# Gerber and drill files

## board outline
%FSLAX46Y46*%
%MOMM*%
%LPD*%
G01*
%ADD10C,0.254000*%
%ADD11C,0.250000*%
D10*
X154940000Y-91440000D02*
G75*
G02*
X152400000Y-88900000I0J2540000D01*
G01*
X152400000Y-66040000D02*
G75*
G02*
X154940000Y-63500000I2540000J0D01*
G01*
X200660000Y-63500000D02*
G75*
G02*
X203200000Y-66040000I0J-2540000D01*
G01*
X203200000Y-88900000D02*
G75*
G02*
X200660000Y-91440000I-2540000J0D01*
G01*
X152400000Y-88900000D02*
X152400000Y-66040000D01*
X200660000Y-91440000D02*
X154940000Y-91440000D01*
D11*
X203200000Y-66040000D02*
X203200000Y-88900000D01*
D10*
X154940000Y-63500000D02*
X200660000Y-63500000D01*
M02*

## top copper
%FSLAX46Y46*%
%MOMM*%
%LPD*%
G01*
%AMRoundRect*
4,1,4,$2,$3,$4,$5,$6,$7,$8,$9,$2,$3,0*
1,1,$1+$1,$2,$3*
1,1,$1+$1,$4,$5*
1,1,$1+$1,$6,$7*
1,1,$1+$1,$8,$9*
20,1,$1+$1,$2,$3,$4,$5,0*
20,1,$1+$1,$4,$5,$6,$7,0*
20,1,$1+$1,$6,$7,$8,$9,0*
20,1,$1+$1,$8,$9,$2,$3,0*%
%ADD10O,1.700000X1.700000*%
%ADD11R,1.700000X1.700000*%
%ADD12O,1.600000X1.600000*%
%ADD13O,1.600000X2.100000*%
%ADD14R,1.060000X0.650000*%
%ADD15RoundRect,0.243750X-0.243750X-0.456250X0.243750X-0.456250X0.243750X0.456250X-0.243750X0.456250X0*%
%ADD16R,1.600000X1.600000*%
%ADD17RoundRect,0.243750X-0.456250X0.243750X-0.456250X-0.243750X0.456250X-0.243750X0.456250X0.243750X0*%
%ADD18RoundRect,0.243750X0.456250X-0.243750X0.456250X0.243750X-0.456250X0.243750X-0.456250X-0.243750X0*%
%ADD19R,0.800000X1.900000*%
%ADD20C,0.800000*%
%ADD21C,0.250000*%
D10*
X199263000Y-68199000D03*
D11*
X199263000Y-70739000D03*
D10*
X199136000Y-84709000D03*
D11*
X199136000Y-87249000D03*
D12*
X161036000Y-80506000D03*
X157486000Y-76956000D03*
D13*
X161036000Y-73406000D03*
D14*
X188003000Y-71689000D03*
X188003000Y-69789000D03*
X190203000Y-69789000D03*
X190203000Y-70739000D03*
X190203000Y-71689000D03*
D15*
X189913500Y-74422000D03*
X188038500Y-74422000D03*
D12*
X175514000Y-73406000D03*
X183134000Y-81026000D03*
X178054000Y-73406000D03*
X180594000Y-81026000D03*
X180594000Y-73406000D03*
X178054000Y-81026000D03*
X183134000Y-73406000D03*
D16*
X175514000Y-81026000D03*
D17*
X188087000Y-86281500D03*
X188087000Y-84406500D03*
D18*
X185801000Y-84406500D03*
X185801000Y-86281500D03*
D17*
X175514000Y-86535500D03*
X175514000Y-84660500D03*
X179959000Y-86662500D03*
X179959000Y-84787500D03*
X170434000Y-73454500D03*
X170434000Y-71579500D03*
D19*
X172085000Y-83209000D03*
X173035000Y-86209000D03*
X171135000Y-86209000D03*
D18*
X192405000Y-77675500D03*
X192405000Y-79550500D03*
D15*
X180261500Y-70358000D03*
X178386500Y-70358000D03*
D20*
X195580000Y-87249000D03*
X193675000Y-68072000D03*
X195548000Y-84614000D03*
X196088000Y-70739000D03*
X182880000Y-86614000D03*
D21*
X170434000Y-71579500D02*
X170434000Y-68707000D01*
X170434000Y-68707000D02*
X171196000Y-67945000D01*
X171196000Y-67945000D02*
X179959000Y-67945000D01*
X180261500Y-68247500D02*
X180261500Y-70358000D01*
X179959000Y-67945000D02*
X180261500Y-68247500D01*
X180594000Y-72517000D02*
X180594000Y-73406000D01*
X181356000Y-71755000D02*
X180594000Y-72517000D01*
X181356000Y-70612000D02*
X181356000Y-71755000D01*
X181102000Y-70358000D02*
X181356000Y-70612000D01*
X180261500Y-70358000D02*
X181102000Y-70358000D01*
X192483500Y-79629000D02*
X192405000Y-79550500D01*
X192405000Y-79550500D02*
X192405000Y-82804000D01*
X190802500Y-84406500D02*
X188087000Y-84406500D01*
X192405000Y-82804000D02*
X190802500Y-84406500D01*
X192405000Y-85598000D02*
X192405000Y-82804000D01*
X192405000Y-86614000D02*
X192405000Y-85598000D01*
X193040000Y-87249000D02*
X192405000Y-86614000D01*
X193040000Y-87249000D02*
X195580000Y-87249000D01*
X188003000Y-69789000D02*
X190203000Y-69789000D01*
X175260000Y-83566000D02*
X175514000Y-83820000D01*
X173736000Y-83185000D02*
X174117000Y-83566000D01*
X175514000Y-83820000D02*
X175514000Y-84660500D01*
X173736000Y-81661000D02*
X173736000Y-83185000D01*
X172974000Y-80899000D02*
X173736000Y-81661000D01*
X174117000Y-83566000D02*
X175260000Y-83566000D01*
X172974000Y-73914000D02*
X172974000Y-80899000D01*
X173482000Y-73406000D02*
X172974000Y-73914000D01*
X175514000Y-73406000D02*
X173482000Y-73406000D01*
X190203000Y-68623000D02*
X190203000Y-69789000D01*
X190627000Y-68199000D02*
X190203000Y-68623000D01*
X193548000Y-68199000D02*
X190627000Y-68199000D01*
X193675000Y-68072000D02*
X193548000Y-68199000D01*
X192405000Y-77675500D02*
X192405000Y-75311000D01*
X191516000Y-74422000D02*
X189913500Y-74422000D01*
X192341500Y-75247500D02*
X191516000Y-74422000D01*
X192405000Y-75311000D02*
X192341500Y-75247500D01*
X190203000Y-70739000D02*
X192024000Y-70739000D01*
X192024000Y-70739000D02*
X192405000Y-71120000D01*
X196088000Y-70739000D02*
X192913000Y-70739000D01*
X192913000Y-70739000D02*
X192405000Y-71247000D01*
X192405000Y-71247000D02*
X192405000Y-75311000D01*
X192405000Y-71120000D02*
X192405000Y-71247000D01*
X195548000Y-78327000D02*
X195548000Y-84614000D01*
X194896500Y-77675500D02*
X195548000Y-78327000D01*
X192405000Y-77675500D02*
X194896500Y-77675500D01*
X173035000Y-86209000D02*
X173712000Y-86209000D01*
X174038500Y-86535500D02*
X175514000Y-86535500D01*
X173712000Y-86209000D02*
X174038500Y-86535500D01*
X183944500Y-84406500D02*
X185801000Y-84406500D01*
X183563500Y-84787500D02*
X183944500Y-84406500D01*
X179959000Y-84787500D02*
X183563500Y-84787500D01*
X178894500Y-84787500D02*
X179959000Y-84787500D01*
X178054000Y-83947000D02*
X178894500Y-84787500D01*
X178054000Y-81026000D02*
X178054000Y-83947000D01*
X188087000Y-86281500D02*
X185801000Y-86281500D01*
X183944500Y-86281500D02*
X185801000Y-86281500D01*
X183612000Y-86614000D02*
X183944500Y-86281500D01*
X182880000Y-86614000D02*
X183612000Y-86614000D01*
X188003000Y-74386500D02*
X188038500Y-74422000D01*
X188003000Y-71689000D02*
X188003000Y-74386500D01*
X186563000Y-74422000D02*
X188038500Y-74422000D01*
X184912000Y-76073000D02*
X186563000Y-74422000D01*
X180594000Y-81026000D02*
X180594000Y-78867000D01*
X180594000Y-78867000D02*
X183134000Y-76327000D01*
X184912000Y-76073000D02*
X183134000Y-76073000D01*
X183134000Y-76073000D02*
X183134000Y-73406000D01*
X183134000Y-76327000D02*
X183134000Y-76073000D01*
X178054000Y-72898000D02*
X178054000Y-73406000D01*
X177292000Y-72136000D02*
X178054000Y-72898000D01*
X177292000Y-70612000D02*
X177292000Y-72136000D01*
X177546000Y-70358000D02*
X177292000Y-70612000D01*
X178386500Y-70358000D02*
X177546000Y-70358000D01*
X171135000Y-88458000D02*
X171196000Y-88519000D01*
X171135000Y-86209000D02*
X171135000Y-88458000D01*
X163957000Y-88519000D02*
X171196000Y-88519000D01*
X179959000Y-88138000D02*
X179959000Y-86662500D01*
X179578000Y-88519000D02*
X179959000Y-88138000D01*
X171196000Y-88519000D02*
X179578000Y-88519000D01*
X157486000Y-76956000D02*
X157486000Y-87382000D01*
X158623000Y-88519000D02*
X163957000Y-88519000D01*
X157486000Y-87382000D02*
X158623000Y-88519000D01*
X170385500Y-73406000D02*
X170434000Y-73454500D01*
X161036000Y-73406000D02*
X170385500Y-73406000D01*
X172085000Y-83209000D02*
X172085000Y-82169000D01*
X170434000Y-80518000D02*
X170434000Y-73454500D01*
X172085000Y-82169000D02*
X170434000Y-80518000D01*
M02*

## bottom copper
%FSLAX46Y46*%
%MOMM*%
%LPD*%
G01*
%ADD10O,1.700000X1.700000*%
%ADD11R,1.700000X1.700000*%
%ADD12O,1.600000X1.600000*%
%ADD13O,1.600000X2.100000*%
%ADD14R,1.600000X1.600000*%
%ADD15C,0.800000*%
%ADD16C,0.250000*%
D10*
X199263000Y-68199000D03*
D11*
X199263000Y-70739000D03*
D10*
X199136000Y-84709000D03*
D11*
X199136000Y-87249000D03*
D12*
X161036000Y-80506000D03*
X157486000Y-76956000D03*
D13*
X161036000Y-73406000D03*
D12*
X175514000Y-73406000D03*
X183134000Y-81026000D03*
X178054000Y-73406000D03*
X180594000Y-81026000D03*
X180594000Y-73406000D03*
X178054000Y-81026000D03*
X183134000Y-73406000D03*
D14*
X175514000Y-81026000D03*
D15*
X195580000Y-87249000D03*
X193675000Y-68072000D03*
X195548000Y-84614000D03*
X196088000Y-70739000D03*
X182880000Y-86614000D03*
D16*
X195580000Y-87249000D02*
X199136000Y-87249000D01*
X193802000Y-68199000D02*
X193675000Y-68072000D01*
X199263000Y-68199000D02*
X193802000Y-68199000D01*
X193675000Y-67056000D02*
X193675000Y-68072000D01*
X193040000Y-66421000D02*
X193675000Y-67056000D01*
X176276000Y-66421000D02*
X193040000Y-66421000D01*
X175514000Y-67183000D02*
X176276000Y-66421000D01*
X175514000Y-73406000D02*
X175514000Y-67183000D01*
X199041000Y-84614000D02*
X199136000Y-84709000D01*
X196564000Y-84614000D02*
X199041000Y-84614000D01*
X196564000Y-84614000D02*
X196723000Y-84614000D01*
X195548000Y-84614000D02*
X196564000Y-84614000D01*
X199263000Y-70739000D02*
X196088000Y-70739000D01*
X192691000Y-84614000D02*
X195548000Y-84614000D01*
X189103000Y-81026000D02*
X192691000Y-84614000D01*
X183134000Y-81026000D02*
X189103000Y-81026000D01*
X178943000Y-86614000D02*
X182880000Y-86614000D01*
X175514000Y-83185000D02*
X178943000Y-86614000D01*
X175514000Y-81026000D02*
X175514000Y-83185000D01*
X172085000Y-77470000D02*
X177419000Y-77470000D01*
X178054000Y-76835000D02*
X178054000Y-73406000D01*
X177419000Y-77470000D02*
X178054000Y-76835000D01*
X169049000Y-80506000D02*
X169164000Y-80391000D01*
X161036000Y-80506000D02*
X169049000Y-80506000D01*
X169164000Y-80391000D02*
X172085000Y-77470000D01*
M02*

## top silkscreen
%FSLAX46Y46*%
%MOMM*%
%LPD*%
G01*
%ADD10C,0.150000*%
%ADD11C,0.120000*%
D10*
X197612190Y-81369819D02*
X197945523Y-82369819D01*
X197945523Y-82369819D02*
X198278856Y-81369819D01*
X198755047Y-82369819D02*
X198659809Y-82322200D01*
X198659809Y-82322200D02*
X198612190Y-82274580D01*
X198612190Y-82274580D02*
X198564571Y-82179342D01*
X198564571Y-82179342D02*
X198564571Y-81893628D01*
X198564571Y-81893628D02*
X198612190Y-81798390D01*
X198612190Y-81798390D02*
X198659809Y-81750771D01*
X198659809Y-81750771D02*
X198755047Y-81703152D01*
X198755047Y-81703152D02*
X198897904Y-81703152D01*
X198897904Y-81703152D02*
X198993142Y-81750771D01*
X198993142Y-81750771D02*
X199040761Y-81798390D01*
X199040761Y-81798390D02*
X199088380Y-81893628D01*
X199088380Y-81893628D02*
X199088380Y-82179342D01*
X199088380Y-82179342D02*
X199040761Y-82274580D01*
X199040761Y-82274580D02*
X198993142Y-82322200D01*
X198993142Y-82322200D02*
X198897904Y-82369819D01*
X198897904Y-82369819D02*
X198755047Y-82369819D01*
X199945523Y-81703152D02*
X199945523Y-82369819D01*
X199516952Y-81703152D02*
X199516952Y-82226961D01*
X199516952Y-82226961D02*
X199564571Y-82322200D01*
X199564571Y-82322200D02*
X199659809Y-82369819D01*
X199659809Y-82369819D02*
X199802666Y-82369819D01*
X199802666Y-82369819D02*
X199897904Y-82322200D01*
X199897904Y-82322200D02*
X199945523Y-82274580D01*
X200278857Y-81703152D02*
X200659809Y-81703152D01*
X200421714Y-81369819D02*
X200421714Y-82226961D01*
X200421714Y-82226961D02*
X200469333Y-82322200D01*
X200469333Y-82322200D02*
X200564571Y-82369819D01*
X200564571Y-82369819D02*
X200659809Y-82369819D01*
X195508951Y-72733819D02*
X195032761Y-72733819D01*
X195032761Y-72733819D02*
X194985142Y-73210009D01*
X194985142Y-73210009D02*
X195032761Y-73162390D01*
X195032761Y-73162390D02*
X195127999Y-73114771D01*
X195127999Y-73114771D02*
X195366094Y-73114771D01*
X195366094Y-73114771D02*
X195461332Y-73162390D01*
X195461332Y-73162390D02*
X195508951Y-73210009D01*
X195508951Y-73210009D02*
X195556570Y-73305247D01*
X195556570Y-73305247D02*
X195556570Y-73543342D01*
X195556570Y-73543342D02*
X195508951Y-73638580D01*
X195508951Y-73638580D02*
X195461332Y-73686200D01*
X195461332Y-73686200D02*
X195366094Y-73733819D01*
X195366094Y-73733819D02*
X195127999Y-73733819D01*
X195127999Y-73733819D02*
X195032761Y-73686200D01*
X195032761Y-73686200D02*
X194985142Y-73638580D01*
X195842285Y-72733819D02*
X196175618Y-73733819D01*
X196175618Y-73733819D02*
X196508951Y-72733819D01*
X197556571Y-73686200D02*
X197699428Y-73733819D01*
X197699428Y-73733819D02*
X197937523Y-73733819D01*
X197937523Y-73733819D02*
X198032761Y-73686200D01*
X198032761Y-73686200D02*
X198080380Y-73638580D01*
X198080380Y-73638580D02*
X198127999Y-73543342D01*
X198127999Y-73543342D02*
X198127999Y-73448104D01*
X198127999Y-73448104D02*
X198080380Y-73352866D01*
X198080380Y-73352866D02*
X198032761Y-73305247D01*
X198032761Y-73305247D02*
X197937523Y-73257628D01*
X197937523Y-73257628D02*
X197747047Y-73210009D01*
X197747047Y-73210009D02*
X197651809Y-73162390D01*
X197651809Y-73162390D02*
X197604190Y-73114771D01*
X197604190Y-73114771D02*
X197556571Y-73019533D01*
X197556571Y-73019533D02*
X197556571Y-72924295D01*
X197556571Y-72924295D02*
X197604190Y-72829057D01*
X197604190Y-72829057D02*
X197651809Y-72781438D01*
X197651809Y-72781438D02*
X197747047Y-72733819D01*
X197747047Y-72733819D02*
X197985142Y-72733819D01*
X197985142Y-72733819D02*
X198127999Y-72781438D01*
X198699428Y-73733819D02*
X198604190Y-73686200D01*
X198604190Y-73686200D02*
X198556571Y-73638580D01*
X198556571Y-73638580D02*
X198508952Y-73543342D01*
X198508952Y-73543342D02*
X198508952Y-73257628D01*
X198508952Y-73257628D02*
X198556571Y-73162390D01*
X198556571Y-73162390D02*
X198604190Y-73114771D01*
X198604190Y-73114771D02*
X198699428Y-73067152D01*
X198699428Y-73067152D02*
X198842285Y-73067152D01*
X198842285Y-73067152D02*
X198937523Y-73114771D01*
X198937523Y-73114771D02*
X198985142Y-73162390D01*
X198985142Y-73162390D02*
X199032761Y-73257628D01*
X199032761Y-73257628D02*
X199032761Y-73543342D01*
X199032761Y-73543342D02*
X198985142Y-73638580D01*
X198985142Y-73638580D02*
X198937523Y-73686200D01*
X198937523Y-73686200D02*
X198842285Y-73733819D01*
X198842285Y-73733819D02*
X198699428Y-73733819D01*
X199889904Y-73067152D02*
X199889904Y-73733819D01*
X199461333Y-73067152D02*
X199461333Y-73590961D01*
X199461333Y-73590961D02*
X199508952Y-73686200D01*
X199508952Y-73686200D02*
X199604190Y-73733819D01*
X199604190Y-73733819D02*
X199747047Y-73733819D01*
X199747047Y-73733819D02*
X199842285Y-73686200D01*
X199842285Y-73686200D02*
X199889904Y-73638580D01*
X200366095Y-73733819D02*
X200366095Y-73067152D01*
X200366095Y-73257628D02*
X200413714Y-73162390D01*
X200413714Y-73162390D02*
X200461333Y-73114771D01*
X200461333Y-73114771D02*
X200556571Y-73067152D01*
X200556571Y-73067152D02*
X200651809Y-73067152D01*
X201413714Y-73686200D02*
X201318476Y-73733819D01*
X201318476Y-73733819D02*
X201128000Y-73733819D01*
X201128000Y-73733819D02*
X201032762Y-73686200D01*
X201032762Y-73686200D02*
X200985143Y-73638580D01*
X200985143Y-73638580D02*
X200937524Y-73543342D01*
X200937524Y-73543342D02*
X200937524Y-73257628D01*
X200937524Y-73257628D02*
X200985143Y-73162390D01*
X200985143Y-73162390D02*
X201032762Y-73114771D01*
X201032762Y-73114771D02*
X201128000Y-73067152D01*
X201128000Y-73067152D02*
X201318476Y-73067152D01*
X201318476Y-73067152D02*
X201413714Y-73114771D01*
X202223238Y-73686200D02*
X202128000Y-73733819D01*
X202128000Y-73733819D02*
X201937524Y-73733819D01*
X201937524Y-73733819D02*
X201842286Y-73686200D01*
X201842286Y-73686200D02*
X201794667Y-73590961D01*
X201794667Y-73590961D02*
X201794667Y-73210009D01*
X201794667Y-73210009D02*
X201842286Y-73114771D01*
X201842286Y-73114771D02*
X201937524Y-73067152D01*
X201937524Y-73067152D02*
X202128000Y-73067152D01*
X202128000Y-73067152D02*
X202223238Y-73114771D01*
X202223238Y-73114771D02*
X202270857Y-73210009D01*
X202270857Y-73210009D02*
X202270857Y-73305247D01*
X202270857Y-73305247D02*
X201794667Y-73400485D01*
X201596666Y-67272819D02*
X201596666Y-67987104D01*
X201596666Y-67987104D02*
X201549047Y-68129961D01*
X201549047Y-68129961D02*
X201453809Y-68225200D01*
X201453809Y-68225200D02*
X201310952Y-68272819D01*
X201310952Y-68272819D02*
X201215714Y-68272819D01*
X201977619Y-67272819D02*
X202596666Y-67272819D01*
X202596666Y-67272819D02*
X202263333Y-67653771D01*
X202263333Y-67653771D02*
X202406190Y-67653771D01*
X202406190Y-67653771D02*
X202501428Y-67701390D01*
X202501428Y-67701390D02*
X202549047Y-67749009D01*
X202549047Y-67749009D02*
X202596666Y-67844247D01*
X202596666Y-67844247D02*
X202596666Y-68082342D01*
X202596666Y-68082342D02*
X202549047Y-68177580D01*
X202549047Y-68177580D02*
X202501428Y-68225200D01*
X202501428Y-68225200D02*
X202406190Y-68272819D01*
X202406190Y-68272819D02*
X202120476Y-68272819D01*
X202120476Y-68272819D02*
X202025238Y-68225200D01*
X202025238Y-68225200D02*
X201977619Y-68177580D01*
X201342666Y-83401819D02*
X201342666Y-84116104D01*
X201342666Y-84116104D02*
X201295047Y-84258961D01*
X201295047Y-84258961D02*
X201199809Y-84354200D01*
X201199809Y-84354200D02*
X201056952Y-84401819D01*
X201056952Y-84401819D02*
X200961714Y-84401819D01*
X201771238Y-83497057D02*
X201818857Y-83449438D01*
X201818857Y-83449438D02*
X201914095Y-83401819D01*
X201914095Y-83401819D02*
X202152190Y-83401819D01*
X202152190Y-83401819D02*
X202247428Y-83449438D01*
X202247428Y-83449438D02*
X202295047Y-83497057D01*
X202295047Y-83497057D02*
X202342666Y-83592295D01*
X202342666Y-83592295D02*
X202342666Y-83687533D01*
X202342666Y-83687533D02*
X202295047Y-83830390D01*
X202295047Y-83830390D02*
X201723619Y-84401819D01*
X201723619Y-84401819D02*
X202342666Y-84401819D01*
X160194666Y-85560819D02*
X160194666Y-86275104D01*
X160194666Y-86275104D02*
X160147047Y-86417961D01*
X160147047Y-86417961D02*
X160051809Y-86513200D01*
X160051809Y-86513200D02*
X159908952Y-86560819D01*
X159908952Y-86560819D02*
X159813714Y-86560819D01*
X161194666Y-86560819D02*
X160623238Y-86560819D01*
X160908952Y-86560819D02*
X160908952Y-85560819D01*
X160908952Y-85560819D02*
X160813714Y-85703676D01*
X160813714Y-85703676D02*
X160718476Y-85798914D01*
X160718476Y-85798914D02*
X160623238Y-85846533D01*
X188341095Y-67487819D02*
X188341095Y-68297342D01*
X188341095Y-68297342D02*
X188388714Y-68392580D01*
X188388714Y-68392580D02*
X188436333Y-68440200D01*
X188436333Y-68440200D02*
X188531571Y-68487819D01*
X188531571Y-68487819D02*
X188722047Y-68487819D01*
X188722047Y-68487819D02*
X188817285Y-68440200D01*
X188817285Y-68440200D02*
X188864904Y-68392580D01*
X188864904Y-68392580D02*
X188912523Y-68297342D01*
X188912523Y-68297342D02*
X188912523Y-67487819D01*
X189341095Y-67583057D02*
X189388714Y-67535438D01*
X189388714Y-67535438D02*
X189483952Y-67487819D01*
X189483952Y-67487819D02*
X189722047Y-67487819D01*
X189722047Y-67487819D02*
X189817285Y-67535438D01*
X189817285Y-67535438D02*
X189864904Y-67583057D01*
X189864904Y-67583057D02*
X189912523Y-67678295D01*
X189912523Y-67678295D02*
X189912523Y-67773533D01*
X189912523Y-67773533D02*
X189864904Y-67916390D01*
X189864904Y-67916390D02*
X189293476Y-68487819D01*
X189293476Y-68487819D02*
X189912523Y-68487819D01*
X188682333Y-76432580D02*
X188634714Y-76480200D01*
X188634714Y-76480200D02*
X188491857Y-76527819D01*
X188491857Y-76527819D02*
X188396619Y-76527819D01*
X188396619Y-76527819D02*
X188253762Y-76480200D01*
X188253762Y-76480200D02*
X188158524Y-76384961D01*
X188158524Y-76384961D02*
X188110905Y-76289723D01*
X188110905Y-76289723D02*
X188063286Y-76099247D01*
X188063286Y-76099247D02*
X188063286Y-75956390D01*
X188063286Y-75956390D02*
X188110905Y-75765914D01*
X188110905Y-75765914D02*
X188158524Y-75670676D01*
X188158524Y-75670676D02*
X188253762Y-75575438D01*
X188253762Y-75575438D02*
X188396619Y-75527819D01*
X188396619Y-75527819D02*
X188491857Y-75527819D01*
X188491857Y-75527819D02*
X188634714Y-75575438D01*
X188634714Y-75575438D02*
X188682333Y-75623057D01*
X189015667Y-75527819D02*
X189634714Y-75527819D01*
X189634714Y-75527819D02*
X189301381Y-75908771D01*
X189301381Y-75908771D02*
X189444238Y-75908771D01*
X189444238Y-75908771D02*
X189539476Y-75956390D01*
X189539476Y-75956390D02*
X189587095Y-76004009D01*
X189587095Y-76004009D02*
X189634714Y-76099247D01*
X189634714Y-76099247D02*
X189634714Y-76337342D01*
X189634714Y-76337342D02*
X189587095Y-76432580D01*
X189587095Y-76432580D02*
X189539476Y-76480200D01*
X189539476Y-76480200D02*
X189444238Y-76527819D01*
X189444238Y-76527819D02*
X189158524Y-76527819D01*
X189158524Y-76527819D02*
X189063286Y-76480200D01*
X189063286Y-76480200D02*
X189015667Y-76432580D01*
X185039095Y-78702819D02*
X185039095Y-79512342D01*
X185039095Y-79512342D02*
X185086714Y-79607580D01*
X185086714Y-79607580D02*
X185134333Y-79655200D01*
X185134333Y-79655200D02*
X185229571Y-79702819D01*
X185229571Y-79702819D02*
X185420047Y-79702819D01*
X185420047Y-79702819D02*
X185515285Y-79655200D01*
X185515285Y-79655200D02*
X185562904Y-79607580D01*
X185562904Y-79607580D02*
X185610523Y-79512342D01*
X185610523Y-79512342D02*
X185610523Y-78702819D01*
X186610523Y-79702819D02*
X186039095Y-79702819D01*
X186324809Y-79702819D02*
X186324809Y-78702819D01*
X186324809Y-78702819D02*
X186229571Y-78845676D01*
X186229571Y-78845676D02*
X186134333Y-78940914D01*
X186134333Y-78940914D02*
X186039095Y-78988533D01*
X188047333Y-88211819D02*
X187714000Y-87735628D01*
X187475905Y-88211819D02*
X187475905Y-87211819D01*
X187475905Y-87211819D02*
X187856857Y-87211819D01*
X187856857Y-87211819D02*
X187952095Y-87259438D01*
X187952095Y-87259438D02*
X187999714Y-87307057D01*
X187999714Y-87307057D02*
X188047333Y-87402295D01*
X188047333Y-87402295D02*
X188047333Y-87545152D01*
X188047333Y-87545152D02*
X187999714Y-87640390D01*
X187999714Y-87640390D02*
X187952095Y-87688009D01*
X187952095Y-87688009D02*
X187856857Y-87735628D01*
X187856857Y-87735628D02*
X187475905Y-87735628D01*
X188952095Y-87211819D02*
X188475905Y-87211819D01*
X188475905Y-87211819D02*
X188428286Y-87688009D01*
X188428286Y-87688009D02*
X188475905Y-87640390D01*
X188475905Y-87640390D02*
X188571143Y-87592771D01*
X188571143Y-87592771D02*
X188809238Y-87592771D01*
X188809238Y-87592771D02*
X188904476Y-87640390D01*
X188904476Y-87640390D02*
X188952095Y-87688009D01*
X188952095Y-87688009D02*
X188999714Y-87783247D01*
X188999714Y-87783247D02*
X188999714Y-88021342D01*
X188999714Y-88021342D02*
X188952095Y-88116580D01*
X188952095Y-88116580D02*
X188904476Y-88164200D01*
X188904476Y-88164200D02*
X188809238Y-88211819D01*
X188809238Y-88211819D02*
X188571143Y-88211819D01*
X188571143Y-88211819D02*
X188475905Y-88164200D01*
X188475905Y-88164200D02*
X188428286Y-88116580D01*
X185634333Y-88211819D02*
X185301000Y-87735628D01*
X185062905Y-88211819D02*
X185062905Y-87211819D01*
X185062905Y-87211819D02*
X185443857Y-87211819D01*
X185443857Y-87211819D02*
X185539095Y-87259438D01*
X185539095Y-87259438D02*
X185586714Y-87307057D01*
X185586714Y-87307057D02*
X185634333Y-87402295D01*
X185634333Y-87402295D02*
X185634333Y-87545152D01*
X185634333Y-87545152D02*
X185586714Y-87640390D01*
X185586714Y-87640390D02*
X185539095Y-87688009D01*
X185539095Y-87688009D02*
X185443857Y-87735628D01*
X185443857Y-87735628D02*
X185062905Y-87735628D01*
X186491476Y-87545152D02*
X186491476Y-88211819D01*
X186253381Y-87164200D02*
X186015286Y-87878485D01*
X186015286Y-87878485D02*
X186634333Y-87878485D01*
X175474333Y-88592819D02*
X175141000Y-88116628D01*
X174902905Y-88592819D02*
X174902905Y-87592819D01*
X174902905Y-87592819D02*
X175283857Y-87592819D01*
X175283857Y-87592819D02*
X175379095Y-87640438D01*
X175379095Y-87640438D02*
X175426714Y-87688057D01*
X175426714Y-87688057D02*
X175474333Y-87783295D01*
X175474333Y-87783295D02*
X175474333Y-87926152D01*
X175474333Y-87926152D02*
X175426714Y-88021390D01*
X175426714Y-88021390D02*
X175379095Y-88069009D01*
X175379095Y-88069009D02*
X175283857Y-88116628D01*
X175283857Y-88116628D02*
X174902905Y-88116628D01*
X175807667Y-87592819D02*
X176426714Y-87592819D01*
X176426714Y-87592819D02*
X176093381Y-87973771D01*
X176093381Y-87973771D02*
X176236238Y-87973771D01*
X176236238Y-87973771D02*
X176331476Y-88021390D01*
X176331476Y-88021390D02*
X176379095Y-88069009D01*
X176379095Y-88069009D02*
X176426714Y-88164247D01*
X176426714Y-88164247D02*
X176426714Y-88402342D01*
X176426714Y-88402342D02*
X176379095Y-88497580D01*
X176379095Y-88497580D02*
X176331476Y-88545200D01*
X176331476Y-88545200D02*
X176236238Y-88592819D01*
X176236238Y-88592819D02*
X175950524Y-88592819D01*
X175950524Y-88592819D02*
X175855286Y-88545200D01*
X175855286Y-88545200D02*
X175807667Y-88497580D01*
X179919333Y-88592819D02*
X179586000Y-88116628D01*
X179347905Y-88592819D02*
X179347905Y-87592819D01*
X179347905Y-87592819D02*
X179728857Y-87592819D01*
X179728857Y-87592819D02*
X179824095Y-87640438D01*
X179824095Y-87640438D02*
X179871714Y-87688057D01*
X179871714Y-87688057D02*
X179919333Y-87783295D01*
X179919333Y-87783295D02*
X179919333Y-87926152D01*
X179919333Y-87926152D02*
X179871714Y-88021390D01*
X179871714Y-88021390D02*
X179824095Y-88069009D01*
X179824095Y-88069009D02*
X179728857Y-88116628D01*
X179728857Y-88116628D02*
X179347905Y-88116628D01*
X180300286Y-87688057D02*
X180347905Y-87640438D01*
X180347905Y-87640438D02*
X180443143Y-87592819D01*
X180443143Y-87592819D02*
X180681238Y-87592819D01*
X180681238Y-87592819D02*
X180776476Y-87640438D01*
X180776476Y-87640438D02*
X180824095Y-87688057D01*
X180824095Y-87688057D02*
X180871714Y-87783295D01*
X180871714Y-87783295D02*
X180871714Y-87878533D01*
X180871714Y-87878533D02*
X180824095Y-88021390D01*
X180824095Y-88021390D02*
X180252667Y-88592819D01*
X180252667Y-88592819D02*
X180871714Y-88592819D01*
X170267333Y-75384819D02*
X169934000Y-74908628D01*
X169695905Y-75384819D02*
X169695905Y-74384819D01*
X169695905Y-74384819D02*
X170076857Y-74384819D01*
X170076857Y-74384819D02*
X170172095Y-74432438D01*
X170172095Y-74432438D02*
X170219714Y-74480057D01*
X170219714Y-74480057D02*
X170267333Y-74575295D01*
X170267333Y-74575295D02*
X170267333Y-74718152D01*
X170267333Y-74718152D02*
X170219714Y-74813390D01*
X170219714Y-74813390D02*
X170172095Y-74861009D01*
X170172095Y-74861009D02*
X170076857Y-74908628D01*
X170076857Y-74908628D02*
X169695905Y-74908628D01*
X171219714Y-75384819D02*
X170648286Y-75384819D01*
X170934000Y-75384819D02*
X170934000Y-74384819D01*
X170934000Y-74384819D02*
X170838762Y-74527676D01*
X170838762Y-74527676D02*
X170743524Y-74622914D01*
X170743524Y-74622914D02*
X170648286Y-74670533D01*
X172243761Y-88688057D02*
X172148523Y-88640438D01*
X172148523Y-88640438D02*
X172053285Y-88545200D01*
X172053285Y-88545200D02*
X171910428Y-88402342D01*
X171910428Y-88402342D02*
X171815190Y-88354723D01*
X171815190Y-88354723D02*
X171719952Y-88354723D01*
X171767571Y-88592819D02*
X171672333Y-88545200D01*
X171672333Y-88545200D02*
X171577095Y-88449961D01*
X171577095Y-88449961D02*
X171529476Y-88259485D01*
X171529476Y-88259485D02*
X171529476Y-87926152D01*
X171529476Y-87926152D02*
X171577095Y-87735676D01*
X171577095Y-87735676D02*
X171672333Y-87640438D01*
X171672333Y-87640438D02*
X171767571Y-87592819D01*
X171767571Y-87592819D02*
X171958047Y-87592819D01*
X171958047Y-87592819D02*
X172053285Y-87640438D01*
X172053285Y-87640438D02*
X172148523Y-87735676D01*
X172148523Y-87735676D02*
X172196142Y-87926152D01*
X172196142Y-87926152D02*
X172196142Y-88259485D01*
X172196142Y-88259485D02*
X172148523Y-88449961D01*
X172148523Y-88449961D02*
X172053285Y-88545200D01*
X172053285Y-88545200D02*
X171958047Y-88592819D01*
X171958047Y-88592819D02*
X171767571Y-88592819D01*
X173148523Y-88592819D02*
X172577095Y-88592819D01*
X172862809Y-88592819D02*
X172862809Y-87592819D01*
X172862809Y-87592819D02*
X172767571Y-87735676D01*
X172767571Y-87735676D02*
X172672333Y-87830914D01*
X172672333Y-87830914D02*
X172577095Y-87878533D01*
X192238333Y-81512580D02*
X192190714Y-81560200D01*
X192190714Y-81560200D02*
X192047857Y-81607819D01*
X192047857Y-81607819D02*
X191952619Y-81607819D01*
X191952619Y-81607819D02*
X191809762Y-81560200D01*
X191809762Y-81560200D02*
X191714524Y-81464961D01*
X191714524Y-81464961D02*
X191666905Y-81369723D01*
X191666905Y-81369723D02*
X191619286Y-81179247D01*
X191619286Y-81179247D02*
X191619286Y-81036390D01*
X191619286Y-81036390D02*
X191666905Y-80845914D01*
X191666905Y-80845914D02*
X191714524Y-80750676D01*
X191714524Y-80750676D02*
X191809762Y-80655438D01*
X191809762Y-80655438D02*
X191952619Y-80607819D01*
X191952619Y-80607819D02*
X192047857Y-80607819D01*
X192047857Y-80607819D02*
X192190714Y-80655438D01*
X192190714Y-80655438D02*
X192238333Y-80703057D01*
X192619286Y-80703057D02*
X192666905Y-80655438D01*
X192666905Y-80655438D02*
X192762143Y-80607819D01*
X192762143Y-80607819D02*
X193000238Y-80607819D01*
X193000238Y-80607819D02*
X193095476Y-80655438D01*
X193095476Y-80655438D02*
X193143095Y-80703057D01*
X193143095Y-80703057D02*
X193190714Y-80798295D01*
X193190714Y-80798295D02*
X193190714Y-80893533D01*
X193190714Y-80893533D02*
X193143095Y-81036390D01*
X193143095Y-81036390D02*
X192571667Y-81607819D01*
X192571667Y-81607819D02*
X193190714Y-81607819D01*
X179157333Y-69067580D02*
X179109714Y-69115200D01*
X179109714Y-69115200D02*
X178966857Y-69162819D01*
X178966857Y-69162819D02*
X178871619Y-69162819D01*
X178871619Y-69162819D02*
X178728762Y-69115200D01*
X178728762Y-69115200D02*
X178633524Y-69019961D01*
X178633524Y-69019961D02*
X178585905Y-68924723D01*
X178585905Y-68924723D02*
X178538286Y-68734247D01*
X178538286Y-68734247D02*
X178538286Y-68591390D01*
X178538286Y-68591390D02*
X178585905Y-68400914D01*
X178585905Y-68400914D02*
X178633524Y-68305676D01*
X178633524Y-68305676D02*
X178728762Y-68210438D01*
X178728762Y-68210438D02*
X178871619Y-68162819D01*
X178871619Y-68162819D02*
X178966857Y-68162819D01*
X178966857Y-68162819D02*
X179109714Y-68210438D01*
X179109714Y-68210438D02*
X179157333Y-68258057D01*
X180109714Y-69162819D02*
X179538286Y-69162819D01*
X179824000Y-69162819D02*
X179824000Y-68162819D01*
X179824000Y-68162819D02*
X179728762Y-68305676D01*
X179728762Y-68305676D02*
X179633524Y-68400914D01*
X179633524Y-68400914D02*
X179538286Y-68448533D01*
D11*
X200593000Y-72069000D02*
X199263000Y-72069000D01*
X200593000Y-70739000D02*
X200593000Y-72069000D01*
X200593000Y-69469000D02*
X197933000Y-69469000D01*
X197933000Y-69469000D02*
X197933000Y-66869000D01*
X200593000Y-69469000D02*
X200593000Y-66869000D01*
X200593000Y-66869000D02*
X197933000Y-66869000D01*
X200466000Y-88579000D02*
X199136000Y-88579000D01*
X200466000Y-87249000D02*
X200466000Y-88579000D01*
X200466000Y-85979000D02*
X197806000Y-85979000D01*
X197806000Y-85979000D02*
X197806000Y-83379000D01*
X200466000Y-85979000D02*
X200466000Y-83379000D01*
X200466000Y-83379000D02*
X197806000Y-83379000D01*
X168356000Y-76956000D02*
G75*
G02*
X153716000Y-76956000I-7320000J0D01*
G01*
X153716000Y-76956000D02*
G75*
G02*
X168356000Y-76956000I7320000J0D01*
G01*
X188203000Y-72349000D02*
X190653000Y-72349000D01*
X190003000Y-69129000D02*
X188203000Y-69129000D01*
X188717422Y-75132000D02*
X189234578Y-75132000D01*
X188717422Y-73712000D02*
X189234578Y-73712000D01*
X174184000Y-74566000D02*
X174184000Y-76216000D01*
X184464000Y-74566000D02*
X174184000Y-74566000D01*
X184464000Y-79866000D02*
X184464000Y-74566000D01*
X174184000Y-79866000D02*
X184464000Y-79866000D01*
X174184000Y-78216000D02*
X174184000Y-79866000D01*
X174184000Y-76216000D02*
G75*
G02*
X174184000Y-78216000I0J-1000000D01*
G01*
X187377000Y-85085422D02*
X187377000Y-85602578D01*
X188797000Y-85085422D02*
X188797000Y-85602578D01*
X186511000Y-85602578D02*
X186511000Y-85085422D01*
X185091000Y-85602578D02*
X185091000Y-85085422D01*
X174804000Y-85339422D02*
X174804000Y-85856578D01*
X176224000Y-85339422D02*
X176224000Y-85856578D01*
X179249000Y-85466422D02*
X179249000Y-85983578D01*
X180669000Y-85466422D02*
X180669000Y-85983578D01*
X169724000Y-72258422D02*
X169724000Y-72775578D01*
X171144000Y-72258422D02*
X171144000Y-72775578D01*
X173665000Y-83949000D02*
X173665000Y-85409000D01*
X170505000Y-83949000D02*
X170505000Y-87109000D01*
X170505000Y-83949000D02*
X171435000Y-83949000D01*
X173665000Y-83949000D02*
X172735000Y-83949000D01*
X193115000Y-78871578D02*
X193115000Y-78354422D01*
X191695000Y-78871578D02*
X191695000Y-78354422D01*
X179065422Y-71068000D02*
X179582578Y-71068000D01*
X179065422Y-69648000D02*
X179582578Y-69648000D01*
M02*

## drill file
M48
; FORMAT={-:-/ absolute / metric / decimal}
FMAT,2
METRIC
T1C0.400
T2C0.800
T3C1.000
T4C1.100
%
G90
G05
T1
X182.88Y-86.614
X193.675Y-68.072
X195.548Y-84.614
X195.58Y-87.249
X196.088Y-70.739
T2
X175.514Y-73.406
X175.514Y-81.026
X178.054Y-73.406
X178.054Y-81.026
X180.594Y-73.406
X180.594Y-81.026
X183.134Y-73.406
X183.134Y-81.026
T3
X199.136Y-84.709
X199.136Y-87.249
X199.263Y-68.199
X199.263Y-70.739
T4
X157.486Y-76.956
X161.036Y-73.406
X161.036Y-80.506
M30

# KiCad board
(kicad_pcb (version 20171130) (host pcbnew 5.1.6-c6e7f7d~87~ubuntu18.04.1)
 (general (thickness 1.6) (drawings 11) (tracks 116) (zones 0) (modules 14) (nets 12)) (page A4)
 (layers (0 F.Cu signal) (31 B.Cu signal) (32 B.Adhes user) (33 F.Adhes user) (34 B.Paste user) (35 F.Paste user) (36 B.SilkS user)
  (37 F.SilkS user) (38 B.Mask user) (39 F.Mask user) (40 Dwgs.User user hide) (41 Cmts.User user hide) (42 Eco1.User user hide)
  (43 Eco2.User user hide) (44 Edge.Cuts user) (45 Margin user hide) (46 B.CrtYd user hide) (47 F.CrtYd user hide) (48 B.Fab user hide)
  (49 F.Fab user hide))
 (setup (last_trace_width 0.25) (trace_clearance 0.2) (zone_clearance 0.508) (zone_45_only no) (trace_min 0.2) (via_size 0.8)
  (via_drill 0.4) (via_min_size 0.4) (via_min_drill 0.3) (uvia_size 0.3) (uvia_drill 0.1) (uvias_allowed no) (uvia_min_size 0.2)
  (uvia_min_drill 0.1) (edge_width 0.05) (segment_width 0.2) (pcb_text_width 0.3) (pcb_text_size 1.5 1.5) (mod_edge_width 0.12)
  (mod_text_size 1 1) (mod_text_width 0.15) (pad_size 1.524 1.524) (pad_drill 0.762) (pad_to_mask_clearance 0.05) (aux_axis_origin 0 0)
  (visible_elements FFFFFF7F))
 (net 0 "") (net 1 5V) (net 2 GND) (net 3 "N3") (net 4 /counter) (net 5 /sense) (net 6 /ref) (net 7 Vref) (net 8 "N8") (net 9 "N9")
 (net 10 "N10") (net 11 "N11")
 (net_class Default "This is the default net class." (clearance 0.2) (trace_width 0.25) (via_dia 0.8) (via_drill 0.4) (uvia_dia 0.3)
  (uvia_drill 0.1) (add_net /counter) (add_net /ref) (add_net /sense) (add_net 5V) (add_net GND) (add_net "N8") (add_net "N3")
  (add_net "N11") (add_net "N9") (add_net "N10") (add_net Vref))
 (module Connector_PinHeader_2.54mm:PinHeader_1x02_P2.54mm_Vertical (layer F.Cu) (at 199.263 70.739 180)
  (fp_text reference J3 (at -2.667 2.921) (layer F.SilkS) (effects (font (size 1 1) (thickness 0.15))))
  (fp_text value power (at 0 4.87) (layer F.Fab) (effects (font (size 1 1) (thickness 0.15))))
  (fp_line (start -1.33 -1.33) (end 0 -1.33) (layer F.SilkS) (width 0.12))
  (fp_line (start -1.33 0) (end -1.33 -1.33) (layer F.SilkS) (width 0.12))
  (fp_line (start -1.33 1.27) (end 1.33 1.27) (layer F.SilkS) (width 0.12))
  (fp_line (start 1.33 1.27) (end 1.33 3.87) (layer F.SilkS) (width 0.12))
  (fp_line (start -1.33 1.27) (end -1.33 3.87) (layer F.SilkS) (width 0.12))
  (fp_line (start -1.33 3.87) (end 1.33 3.87) (layer F.SilkS) (width 0.12))
  (pad 2 thru_hole oval (at 0 2.54 180) (size 1.7 1.7) (drill 1) (layers *.Cu *.Mask) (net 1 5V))
  (pad 1 thru_hole rect (at 0 0 180) (size 1.7 1.7) (drill 1) (layers *.Cu *.Mask) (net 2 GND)))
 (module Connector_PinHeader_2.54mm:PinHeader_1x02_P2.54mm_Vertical (layer F.Cu) (at 199.136 87.249 180)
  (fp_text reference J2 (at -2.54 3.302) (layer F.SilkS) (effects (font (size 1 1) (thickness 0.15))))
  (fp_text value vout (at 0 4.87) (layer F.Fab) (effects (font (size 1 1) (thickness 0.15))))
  (fp_line (start -1.33 -1.33) (end 0 -1.33) (layer F.SilkS) (width 0.12))
  (fp_line (start -1.33 0) (end -1.33 -1.33) (layer F.SilkS) (width 0.12))
  (fp_line (start -1.33 1.27) (end 1.33 1.27) (layer F.SilkS) (width 0.12))
  (fp_line (start 1.33 1.27) (end 1.33 3.87) (layer F.SilkS) (width 0.12))
  (fp_line (start -1.33 1.27) (end -1.33 3.87) (layer F.SilkS) (width 0.12))
  (fp_line (start -1.33 3.87) (end 1.33 3.87) (layer F.SilkS) (width 0.12))
  (pad 2 thru_hole oval (at 0 2.54 180) (size 1.7 1.7) (drill 1) (layers *.Cu *.Mask) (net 2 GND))
  (pad 1 thru_hole rect (at 0 0 180) (size 1.7 1.7) (drill 1) (layers *.Cu *.Mask) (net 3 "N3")))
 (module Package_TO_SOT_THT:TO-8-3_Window (layer F.Cu) (at 161.036 73.406 270)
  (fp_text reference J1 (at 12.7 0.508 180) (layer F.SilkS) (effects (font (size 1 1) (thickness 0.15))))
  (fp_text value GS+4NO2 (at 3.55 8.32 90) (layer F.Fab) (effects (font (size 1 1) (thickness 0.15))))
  (fp_circle (center 3.55 0) (end 10.87 0) (layer F.SilkS) (width 0.12))
  (pad 3 thru_hole oval (at 7.1 0 270) (size 1.6 1.6) (drill 1.1) (layers *.Cu *.Mask) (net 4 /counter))
  (pad 2 thru_hole oval (at 3.55 3.55 270) (size 1.6 1.6) (drill 1.1) (layers *.Cu *.Mask) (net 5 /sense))
  (pad 1 thru_hole oval (at 0 0 270) (size 2.1 1.6) (drill 1.1) (layers *.Cu *.Mask) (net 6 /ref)))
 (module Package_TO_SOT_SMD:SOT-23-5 (layer F.Cu) (at 189.103 70.739 180)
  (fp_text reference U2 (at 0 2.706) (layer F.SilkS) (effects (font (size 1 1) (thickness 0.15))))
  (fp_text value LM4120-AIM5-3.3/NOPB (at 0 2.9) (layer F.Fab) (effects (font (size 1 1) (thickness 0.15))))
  (fp_line (start 0.9 -1.61) (end -1.55 -1.61) (layer F.SilkS) (width 0.12))
  (fp_line (start -0.9 1.61) (end 0.9 1.61) (layer F.SilkS) (width 0.12))
  (pad 5 smd rect (at 1.1 -0.95 180) (size 1.06 0.65) (layers F.Cu F.Paste F.Mask) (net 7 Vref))
  (pad 4 smd rect (at 1.1 0.95 180) (size 1.06 0.65) (layers F.Cu F.Paste F.Mask) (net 1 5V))
  (pad 3 smd rect (at -1.1 0.95 180) (size 1.06 0.65) (layers F.Cu F.Paste F.Mask) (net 1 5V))
  (pad 2 smd rect (at -1.1 0 180) (size 1.06 0.65) (layers F.Cu F.Paste F.Mask) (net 2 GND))
  (pad 1 smd rect (at -1.1 -0.95 180) (size 1.06 0.65) (layers F.Cu F.Paste F.Mask)))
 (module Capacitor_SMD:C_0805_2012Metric (layer F.Cu) (at 188.976 74.422)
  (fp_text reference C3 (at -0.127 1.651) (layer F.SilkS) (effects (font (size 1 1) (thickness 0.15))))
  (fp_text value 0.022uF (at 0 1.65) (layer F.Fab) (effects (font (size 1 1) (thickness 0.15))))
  (fp_line (start -0.258578 0.71) (end 0.258578 0.71) (layer F.SilkS) (width 0.12))
  (fp_line (start -0.258578 -0.71) (end 0.258578 -0.71) (layer F.SilkS) (width 0.12))
  (pad 2 smd roundrect (at 0.9375 0) (size 0.975 1.4) (layers F.Cu F.Paste F.Mask) (roundrect_rratio 0.25) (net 2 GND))
  (pad 1 smd roundrect (at -0.9375 0) (size 0.975 1.4) (layers F.Cu F.Paste F.Mask) (roundrect_rratio 0.25) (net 7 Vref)))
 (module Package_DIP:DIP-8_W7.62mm (layer F.Cu) (at 175.514 81.026 90)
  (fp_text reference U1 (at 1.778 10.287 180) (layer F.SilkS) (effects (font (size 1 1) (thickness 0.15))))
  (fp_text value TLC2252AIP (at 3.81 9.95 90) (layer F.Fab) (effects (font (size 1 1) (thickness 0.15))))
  (fp_line (start 6.46 -1.33) (end 4.81 -1.33) (layer F.SilkS) (width 0.12))
  (fp_line (start 6.46 8.95) (end 6.46 -1.33) (layer F.SilkS) (width 0.12))
  (fp_line (start 1.16 8.95) (end 6.46 8.95) (layer F.SilkS) (width 0.12))
  (fp_line (start 1.16 -1.33) (end 1.16 8.95) (layer F.SilkS) (width 0.12))
  (fp_line (start 2.81 -1.33) (end 1.16 -1.33) (layer F.SilkS) (width 0.12))
  (fp_arc (start 3.81 -1.33) (end 2.81 -1.33) (angle -180) (layer F.SilkS) (width 0.12))
  (pad 8 thru_hole oval (at 7.62 0 90) (size 1.6 1.6) (drill 0.8) (layers *.Cu *.Mask) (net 1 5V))
  (pad 4 thru_hole oval (at 0 7.62 90) (size 1.6 1.6) (drill 0.8) (layers *.Cu *.Mask) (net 2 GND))
  (pad 7 thru_hole oval (at 7.62 2.54 90) (size 1.6 1.6) (drill 0.8) (layers *.Cu *.Mask) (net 4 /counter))
  (pad 3 thru_hole oval (at 0 5.08 90) (size 1.6 1.6) (drill 0.8) (layers *.Cu *.Mask) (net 7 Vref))
  (pad 6 thru_hole oval (at 7.62 5.08 90) (size 1.6 1.6) (drill 0.8) (layers *.Cu *.Mask) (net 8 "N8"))
  (pad 2 thru_hole oval (at 0 2.54 90) (size 1.6 1.6) (drill 0.8) (layers *.Cu *.Mask) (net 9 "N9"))
  (pad 5 thru_hole oval (at 7.62 7.62 90) (size 1.6 1.6) (drill 0.8) (layers *.Cu *.Mask) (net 7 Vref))
  (pad 1 thru_hole rect (at 0 0 90) (size 1.6 1.6) (drill 0.8) (layers *.Cu *.Mask) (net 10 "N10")))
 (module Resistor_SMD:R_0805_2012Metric (layer F.Cu) (at 188.087 85.344 270)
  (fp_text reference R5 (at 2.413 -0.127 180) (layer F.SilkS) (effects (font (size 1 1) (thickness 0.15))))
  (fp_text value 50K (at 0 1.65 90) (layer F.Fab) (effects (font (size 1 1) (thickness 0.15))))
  (fp_line (start -0.258578 0.71) (end 0.258578 0.71) (layer F.SilkS) (width 0.12))
  (fp_line (start -0.258578 -0.71) (end 0.258578 -0.71) (layer F.SilkS) (width 0.12))
  (pad 2 smd roundrect (at 0.9375 0 270) (size 0.975 1.4) (layers F.Cu F.Paste F.Mask) (roundrect_rratio 0.25) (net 10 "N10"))
  (pad 1 smd roundrect (at -0.9375 0 270) (size 0.975 1.4) (layers F.Cu F.Paste F.Mask) (roundrect_rratio 0.25) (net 3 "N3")))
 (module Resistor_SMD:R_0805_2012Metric (layer F.Cu) (at 185.801 85.344 90)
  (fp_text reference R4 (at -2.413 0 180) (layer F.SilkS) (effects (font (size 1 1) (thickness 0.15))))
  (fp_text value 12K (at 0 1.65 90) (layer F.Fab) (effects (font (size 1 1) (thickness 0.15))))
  (fp_line (start -0.258578 0.71) (end 0.258578 0.71) (layer F.SilkS) (width 0.12))
  (fp_line (start -0.258578 -0.71) (end 0.258578 -0.71) (layer F.SilkS) (width 0.12))
  (pad 2 smd roundrect (at 0.9375 0 90) (size 0.975 1.4) (layers F.Cu F.Paste F.Mask) (roundrect_rratio 0.25) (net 9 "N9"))
  (pad 1 smd roundrect (at -0.9375 0 90) (size 0.975 1.4) (layers F.Cu F.Paste F.Mask) (roundrect_rratio 0.25) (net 10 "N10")))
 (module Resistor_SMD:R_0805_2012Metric (layer F.Cu) (at 175.514 85.598 270)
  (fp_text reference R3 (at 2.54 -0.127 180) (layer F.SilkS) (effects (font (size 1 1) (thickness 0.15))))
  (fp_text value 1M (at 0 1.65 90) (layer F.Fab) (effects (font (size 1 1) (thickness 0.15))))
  (fp_line (start -0.258578 0.71) (end 0.258578 0.71) (layer F.SilkS) (width 0.12))
  (fp_line (start -0.258578 -0.71) (end 0.258578 -0.71) (layer F.SilkS) (width 0.12))
  (pad 2 smd roundrect (at 0.9375 0 270) (size 0.975 1.4) (layers F.Cu F.Paste F.Mask) (roundrect_rratio 0.25) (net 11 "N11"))
  (pad 1 smd roundrect (at -0.9375 0 270) (size 0.975 1.4) (layers F.Cu F.Paste F.Mask) (roundrect_rratio 0.25) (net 1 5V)))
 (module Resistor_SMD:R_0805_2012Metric (layer F.Cu) (at 179.959 85.725 270)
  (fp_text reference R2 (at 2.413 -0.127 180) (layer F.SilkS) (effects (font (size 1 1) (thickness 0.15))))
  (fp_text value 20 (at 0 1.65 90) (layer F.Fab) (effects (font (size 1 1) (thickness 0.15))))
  (fp_line (start -0.258578 0.71) (end 0.258578 0.71) (layer F.SilkS) (width 0.12))
  (fp_line (start -0.258578 -0.71) (end 0.258578 -0.71) (layer F.SilkS) (width 0.12))
  (pad 2 smd roundrect (at 0.9375 0 270) (size 0.975 1.4) (layers F.Cu F.Paste F.Mask) (roundrect_rratio 0.25) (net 5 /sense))
  (pad 1 smd roundrect (at -0.9375 0 270) (size 0.975 1.4) (layers F.Cu F.Paste F.Mask) (roundrect_rratio 0.25) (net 9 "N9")))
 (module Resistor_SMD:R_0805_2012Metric (layer F.Cu) (at 170.434 72.517 270)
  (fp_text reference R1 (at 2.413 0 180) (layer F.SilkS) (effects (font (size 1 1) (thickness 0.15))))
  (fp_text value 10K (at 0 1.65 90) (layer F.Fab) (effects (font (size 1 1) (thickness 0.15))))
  (fp_line (start -0.258578 0.71) (end 0.258578 0.71) (layer F.SilkS) (width 0.12))
  (fp_line (start -0.258578 -0.71) (end 0.258578 -0.71) (layer F.SilkS) (width 0.12))
  (pad 2 smd roundrect (at 0.9375 0 270) (size 0.975 1.4) (layers F.Cu F.Paste F.Mask) (roundrect_rratio 0.25) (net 6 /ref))
  (pad 1 smd roundrect (at -0.9375 0 270) (size 0.975 1.4) (layers F.Cu F.Paste F.Mask) (roundrect_rratio 0.25) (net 8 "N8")))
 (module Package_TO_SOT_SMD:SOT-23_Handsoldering (layer F.Cu) (at 172.085 84.709 90)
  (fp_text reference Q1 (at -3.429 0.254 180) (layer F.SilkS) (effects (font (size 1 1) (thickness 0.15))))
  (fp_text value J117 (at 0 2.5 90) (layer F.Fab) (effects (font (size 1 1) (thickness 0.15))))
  (fp_line (start 0.76 1.58) (end -0.7 1.58) (layer F.SilkS) (width 0.12))
  (fp_line (start 0.76 -1.58) (end -2.4 -1.58) (layer F.SilkS) (width 0.12))
  (fp_line (start 0.76 -1.58) (end 0.76 -0.65) (layer F.SilkS) (width 0.12))
  (fp_line (start 0.76 1.58) (end 0.76 0.65) (layer F.SilkS) (width 0.12))
  (pad 3 smd rect (at 1.5 0 90) (size 1.9 0.8) (layers F.Cu F.Paste F.Mask) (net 6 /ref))
  (pad 2 smd rect (at -1.5 0.95 90) (size 1.9 0.8) (layers F.Cu F.Paste F.Mask) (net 11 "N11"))
  (pad 1 smd rect (at -1.5 -0.95 90) (size 1.9 0.8) (layers F.Cu F.Paste F.Mask) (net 5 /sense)))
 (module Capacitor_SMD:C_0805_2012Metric (layer F.Cu) (at 192.405 78.613 90)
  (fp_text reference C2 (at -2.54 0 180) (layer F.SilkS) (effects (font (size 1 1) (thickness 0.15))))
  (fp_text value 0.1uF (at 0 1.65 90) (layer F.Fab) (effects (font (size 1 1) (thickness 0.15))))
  (fp_line (start -0.258578 0.71) (end 0.258578 0.71) (layer F.SilkS) (width 0.12))
  (fp_line (start -0.258578 -0.71) (end 0.258578 -0.71) (layer F.SilkS) (width 0.12))
  (pad 2 smd roundrect (at 0.9375 0 90) (size 0.975 1.4) (layers F.Cu F.Paste F.Mask) (roundrect_rratio 0.25) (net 2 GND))
  (pad 1 smd roundrect (at -0.9375 0 90) (size 0.975 1.4) (layers F.Cu F.Paste F.Mask) (roundrect_rratio 0.25) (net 3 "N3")))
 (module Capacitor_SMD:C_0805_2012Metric (layer F.Cu) (at 179.324 70.358)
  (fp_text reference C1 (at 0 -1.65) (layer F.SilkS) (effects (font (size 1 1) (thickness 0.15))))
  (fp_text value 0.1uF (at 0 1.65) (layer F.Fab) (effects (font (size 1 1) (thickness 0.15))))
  (fp_line (start -0.258578 0.71) (end 0.258578 0.71) (layer F.SilkS) (width 0.12))
  (fp_line (start -0.258578 -0.71) (end 0.258578 -0.71) (layer F.SilkS) (width 0.12))
  (pad 2 smd roundrect (at 0.9375 0) (size 0.975 1.4) (layers F.Cu F.Paste F.Mask) (roundrect_rratio 0.25) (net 8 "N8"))
  (pad 1 smd roundrect (at -0.9375 0) (size 0.975 1.4) (layers F.Cu F.Paste F.Mask) (roundrect_rratio 0.25) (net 4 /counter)))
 (gr_arc (start 154.94 88.9) (end 152.4 88.9) (angle -90) (layer Edge.Cuts) (width 0.254))
 (gr_arc (start 154.94 66.04) (end 154.94 63.5) (angle -90) (layer Edge.Cuts) (width 0.254))
 (gr_arc (start 200.66 66.04) (end 203.2 66.04) (angle -90) (layer Edge.Cuts) (width 0.254))
 (gr_arc (start 200.66 88.9) (end 200.66 91.44) (angle -90) (layer Edge.Cuts) (width 0.254))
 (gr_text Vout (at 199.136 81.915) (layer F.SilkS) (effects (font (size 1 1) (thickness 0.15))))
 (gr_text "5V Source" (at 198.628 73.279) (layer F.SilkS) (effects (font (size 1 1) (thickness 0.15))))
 (gr_line (start 152.4 88.9) (end 152.4 66.04) (layer Edge.Cuts) (width 0.254))
 (gr_line (start 200.66 91.44) (end 154.94 91.44) (layer Edge.Cuts) (width 0.254))
 (gr_line (start 203.2 66.04) (end 203.2 88.9) (layer Edge.Cuts) (width 0.25))
 (gr_line (start 154.94 63.5) (end 200.66 63.5) (layer Edge.Cuts) (width 0.254))
 (segment (start 170.434 71.5795) (end 170.434 68.707) (width 0.25) (layer F.Cu) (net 8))
 (segment (start 170.434 68.707) (end 171.196 67.945) (width 0.25) (layer F.Cu) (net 8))
 (segment (start 171.196 67.945) (end 179.959 67.945) (width 0.25) (layer F.Cu) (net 8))
 (segment (start 180.2615 68.2475) (end 180.2615 70.358) (width 0.25) (layer F.Cu) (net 8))
 (segment (start 179.959 67.945) (end 180.2615 68.2475) (width 0.25) (layer F.Cu) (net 8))
 (segment (start 180.594 72.517) (end 180.594 73.406) (width 0.25) (layer F.Cu) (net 8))
 (segment (start 181.356 71.755) (end 180.594 72.517) (width 0.25) (layer F.Cu) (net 8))
 (segment (start 181.356 70.612) (end 181.356 71.755) (width 0.25) (layer F.Cu) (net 8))
 (segment (start 181.102 70.358) (end 181.356 70.612) (width 0.25) (layer F.Cu) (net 8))
 (segment (start 180.2615 70.358) (end 181.102 70.358) (width 0.25) (layer F.Cu) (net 8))
 (segment (start 192.4835 79.629) (end 192.405 79.5505) (width 0.25) (layer F.Cu) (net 3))
 (segment (start 192.405 79.5505) (end 192.405 82.804) (width 0.25) (layer F.Cu) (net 3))
 (segment (start 190.8025 84.4065) (end 188.087 84.4065) (width 0.25) (layer F.Cu) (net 3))
 (segment (start 192.405 82.804) (end 190.8025 84.4065) (width 0.25) (layer F.Cu) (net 3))
 (segment (start 192.405 85.598) (end 192.405 82.804) (width 0.25) (layer F.Cu) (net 3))
 (segment (start 192.405 86.614) (end 192.405 85.598) (width 0.25) (layer F.Cu) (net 3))
 (segment (start 193.04 87.249) (end 192.405 86.614) (width 0.25) (layer F.Cu) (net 3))
 (via (at 195.58 87.249) (size 0.8) (drill 0.4) (layers F.Cu B.Cu) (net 3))
 (segment (start 193.04 87.249) (end 195.58 87.249) (width 0.25) (layer F.Cu) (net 3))
 (segment (start 195.58 87.249) (end 199.136 87.249) (width 0.25) (layer B.Cu) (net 3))
 (segment (start 188.003 69.789) (end 190.203 69.789) (width 0.25) (layer F.Cu) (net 1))
 (segment (start 175.26 83.566) (end 175.514 83.82) (width 0.25) (layer F.Cu) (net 1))
 (segment (start 173.736 83.185) (end 174.117 83.566) (width 0.25) (layer F.Cu) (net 1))
 (segment (start 175.514 83.82) (end 175.514 84.6605) (width 0.25) (layer F.Cu) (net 1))
 (segment (start 173.736 81.661) (end 173.736 83.185) (width 0.25) (layer F.Cu) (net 1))
 (segment (start 172.974 80.899) (end 173.736 81.661) (width 0.25) (layer F.Cu) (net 1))
 (segment (start 174.117 83.566) (end 175.26 83.566) (width 0.25) (layer F.Cu) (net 1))
 (segment (start 172.974 73.914) (end 172.974 80.899) (width 0.25) (layer F.Cu) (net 1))
 (segment (start 173.482 73.406) (end 172.974 73.914) (width 0.25) (layer F.Cu) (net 1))
 (segment (start 175.514 73.406) (end 173.482 73.406) (width 0.25) (layer F.Cu) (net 1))
 (via (at 193.675 68.072) (size 0.8) (drill 0.4) (layers F.Cu B.Cu) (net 1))
 (segment (start 193.802 68.199) (end 193.675 68.072) (width 0.25) (layer B.Cu) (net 1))
 (segment (start 199.263 68.199) (end 193.802 68.199) (width 0.25) (layer B.Cu) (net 1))
 (segment (start 190.203 68.623) (end 190.203 69.789) (width 0.25) (layer F.Cu) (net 1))
 (segment (start 190.627 68.199) (end 190.203 68.623) (width 0.25) (layer F.Cu) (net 1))
 (segment (start 193.548 68.199) (end 190.627 68.199) (width 0.25) (layer F.Cu) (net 1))
 (segment (start 193.675 68.072) (end 193.548 68.199) (width 0.25) (layer F.Cu) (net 1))
 (segment (start 193.675 67.056) (end 193.675 68.072) (width 0.25) (layer B.Cu) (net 1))
 (segment (start 193.04 66.421) (end 193.675 67.056) (width 0.25) (layer B.Cu) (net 1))
 (segment (start 176.276 66.421) (end 193.04 66.421) (width 0.25) (layer B.Cu) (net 1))
 (segment (start 175.514 67.183) (end 176.276 66.421) (width 0.25) (layer B.Cu) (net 1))
 (segment (start 175.514 73.406) (end 175.514 67.183) (width 0.25) (layer B.Cu) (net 1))
 (segment (start 192.405 77.6755) (end 192.405 75.311) (width 0.25) (layer F.Cu) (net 2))
 (segment (start 191.516 74.422) (end 189.9135 74.422) (width 0.25) (layer F.Cu) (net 2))
 (segment (start 192.3415 75.2475) (end 191.516 74.422) (width 0.25) (layer F.Cu) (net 2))
 (segment (start 192.405 75.311) (end 192.3415 75.2475) (width 0.25) (layer F.Cu) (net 2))
 (segment (start 190.203 70.739) (end 192.024 70.739) (width 0.25) (layer F.Cu) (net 2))
 (segment (start 192.024 70.739) (end 192.405 71.12) (width 0.25) (layer F.Cu) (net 2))
 (segment (start 199.041 84.614) (end 199.136 84.709) (width 0.25) (layer B.Cu) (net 2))
 (segment (start 196.564 84.614) (end 199.041 84.614) (width 0.25) (layer B.Cu) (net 2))
 (segment (start 196.564 84.614) (end 196.723 84.614) (width 0.25) (layer B.Cu) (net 2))
 (via (at 195.548 84.614) (size 0.8) (drill 0.4) (layers F.Cu B.Cu) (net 2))
 (segment (start 195.548 84.614) (end 196.564 84.614) (width 0.25) (layer B.Cu) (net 2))
 (via (at 196.088 70.739) (size 0.8) (drill 0.4) (layers F.Cu B.Cu) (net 2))
 (segment (start 199.263 70.739) (end 196.088 70.739) (width 0.25) (layer B.Cu) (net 2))
 (segment (start 196.088 70.739) (end 192.913 70.739) (width 0.25) (layer F.Cu) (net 2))
 (segment (start 192.913 70.739) (end 192.405 71.247) (width 0.25) (layer F.Cu) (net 2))
 (segment (start 192.405 71.247) (end 192.405 75.311) (width 0.25) (layer F.Cu) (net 2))
 (segment (start 192.405 71.12) (end 192.405 71.247) (width 0.25) (layer F.Cu) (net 2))
 (segment (start 192.691 84.614) (end 195.548 84.614) (width 0.25) (layer B.Cu) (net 2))
 (segment (start 189.103 81.026) (end 192.691 84.614) (width 0.25) (layer B.Cu) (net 2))
 (segment (start 183.134 81.026) (end 189.103 81.026) (width 0.25) (layer B.Cu) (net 2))
 (segment (start 195.548 78.327) (end 195.548 84.614) (width 0.25) (layer F.Cu) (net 2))
 (segment (start 194.8965 77.6755) (end 195.548 78.327) (width 0.25) (layer F.Cu) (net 2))
 (segment (start 192.405 77.6755) (end 194.8965 77.6755) (width 0.25) (layer F.Cu) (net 2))
 (segment (start 173.035 86.209) (end 173.712 86.209) (width 0.25) (layer F.Cu) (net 11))
 (segment (start 174.0385 86.5355) (end 175.514 86.5355) (width 0.25) (layer F.Cu) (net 11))
 (segment (start 173.712 86.209) (end 174.0385 86.5355) (width 0.25) (layer F.Cu) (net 11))
 (segment (start 183.9445 84.4065) (end 185.801 84.4065) (width 0.25) (layer F.Cu) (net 9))
 (segment (start 183.5635 84.7875) (end 183.9445 84.4065) (width 0.25) (layer F.Cu) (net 9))
 (segment (start 179.959 84.7875) (end 183.5635 84.7875) (width 0.25) (layer F.Cu) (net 9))
 (segment (start 178.8945 84.7875) (end 179.959 84.7875) (width 0.25) (layer F.Cu) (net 9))
 (segment (start 178.054 83.947) (end 178.8945 84.7875) (width 0.25) (layer F.Cu) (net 9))
 (segment (start 178.054 81.026) (end 178.054 83.947) (width 0.25) (layer F.Cu) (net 9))
 (segment (start 188.087 86.2815) (end 185.801 86.2815) (width 0.25) (layer F.Cu) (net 10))
 (segment (start 183.9445 86.2815) (end 185.801 86.2815) (width 0.25) (layer F.Cu) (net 10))
 (via (at 182.88 86.614) (size 0.8) (drill 0.4) (layers F.Cu B.Cu) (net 10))
 (segment (start 183.612 86.614) (end 183.9445 86.2815) (width 0.25) (layer F.Cu) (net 10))
 (segment (start 182.88 86.614) (end 183.612 86.614) (width 0.25) (layer F.Cu) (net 10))
 (segment (start 178.943 86.614) (end 182.88 86.614) (width 0.25) (layer B.Cu) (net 10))
 (segment (start 175.514 83.185) (end 178.943 86.614) (width 0.25) (layer B.Cu) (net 10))
 (segment (start 175.514 81.026) (end 175.514 83.185) (width 0.25) (layer B.Cu) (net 10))
 (segment (start 188.003 74.3865) (end 188.0385 74.422) (width 0.25) (layer F.Cu) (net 7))
 (segment (start 188.003 71.689) (end 188.003 74.3865) (width 0.25) (layer F.Cu) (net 7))
 (segment (start 186.563 74.422) (end 188.0385 74.422) (width 0.25) (layer F.Cu) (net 7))
 (segment (start 184.912 76.073) (end 186.563 74.422) (width 0.25) (layer F.Cu) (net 7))
 (segment (start 180.594 81.026) (end 180.594 78.867) (width 0.25) (layer F.Cu) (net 7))
 (segment (start 180.594 78.867) (end 183.134 76.327) (width 0.25) (layer F.Cu) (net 7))
 (segment (start 184.912 76.073) (end 183.134 76.073) (width 0.25) (layer F.Cu) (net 7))
 (segment (start 183.134 76.073) (end 183.134 73.406) (width 0.25) (layer F.Cu) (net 7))
 (segment (start 183.134 76.327) (end 183.134 76.073) (width 0.25) (layer F.Cu) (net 7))
 (segment (start 172.085 77.47) (end 177.419 77.47) (width 0.25) (layer B.Cu) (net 4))
 (segment (start 178.054 76.835) (end 178.054 73.406) (width 0.25) (layer B.Cu) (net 4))
 (segment (start 177.419 77.47) (end 178.054 76.835) (width 0.25) (layer B.Cu) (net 4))
 (segment (start 169.049 80.506) (end 169.164 80.391) (width 0.25) (layer B.Cu) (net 4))
 (segment (start 161.036 80.506) (end 169.049 80.506) (width 0.25) (layer B.Cu) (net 4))
 (segment (start 169.164 80.391) (end 172.085 77.47) (width 0.25) (layer B.Cu) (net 4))
 (segment (start 178.054 72.898) (end 178.054 73.406) (width 0.25) (layer F.Cu) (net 4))
 (segment (start 177.292 72.136) (end 178.054 72.898) (width 0.25) (layer F.Cu) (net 4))
 (segment (start 177.292 70.612) (end 177.292 72.136) (width 0.25) (layer F.Cu) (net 4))
 (segment (start 177.546 70.358) (end 177.292 70.612) (width 0.25) (layer F.Cu) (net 4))
 (segment (start 178.3865 70.358) (end 177.546 70.358) (width 0.25) (layer F.Cu) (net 4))
 (segment (start 171.135 88.458) (end 171.196 88.519) (width 0.25) (layer F.Cu) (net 5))
 (segment (start 171.135 86.209) (end 171.135 88.458) (width 0.25) (layer F.Cu) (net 5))
 (segment (start 163.957 88.519) (end 171.196 88.519) (width 0.25) (layer F.Cu) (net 5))
 (segment (start 179.959 88.138) (end 179.959 86.6625) (width 0.25) (layer F.Cu) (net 5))
 (segment (start 179.578 88.519) (end 179.959 88.138) (width 0.25) (layer F.Cu) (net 5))
 (segment (start 171.196 88.519) (end 179.578 88.519) (width 0.25) (layer F.Cu) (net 5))
 (segment (start 157.486 76.956) (end 157.486 87.382) (width 0.25) (layer F.Cu) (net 5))
 (segment (start 158.623 88.519) (end 163.957 88.519) (width 0.25) (layer F.Cu) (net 5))
 (segment (start 157.486 87.382) (end 158.623 88.519) (width 0.25) (layer F.Cu) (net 5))
 (segment (start 170.3855 73.406) (end 170.434 73.4545) (width 0.25) (layer F.Cu) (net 6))
 (segment (start 161.036 73.406) (end 170.3855 73.406) (width 0.25) (layer F.Cu) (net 6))
 (segment (start 172.085 83.209) (end 172.085 82.169) (width 0.25) (layer F.Cu) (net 6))
 (segment (start 170.434 80.518) (end 170.434 73.4545) (width 0.25) (layer F.Cu) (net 6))
 (segment (start 172.085 82.169) (end 170.434 80.518) (width 0.25) (layer F.Cu) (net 6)))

